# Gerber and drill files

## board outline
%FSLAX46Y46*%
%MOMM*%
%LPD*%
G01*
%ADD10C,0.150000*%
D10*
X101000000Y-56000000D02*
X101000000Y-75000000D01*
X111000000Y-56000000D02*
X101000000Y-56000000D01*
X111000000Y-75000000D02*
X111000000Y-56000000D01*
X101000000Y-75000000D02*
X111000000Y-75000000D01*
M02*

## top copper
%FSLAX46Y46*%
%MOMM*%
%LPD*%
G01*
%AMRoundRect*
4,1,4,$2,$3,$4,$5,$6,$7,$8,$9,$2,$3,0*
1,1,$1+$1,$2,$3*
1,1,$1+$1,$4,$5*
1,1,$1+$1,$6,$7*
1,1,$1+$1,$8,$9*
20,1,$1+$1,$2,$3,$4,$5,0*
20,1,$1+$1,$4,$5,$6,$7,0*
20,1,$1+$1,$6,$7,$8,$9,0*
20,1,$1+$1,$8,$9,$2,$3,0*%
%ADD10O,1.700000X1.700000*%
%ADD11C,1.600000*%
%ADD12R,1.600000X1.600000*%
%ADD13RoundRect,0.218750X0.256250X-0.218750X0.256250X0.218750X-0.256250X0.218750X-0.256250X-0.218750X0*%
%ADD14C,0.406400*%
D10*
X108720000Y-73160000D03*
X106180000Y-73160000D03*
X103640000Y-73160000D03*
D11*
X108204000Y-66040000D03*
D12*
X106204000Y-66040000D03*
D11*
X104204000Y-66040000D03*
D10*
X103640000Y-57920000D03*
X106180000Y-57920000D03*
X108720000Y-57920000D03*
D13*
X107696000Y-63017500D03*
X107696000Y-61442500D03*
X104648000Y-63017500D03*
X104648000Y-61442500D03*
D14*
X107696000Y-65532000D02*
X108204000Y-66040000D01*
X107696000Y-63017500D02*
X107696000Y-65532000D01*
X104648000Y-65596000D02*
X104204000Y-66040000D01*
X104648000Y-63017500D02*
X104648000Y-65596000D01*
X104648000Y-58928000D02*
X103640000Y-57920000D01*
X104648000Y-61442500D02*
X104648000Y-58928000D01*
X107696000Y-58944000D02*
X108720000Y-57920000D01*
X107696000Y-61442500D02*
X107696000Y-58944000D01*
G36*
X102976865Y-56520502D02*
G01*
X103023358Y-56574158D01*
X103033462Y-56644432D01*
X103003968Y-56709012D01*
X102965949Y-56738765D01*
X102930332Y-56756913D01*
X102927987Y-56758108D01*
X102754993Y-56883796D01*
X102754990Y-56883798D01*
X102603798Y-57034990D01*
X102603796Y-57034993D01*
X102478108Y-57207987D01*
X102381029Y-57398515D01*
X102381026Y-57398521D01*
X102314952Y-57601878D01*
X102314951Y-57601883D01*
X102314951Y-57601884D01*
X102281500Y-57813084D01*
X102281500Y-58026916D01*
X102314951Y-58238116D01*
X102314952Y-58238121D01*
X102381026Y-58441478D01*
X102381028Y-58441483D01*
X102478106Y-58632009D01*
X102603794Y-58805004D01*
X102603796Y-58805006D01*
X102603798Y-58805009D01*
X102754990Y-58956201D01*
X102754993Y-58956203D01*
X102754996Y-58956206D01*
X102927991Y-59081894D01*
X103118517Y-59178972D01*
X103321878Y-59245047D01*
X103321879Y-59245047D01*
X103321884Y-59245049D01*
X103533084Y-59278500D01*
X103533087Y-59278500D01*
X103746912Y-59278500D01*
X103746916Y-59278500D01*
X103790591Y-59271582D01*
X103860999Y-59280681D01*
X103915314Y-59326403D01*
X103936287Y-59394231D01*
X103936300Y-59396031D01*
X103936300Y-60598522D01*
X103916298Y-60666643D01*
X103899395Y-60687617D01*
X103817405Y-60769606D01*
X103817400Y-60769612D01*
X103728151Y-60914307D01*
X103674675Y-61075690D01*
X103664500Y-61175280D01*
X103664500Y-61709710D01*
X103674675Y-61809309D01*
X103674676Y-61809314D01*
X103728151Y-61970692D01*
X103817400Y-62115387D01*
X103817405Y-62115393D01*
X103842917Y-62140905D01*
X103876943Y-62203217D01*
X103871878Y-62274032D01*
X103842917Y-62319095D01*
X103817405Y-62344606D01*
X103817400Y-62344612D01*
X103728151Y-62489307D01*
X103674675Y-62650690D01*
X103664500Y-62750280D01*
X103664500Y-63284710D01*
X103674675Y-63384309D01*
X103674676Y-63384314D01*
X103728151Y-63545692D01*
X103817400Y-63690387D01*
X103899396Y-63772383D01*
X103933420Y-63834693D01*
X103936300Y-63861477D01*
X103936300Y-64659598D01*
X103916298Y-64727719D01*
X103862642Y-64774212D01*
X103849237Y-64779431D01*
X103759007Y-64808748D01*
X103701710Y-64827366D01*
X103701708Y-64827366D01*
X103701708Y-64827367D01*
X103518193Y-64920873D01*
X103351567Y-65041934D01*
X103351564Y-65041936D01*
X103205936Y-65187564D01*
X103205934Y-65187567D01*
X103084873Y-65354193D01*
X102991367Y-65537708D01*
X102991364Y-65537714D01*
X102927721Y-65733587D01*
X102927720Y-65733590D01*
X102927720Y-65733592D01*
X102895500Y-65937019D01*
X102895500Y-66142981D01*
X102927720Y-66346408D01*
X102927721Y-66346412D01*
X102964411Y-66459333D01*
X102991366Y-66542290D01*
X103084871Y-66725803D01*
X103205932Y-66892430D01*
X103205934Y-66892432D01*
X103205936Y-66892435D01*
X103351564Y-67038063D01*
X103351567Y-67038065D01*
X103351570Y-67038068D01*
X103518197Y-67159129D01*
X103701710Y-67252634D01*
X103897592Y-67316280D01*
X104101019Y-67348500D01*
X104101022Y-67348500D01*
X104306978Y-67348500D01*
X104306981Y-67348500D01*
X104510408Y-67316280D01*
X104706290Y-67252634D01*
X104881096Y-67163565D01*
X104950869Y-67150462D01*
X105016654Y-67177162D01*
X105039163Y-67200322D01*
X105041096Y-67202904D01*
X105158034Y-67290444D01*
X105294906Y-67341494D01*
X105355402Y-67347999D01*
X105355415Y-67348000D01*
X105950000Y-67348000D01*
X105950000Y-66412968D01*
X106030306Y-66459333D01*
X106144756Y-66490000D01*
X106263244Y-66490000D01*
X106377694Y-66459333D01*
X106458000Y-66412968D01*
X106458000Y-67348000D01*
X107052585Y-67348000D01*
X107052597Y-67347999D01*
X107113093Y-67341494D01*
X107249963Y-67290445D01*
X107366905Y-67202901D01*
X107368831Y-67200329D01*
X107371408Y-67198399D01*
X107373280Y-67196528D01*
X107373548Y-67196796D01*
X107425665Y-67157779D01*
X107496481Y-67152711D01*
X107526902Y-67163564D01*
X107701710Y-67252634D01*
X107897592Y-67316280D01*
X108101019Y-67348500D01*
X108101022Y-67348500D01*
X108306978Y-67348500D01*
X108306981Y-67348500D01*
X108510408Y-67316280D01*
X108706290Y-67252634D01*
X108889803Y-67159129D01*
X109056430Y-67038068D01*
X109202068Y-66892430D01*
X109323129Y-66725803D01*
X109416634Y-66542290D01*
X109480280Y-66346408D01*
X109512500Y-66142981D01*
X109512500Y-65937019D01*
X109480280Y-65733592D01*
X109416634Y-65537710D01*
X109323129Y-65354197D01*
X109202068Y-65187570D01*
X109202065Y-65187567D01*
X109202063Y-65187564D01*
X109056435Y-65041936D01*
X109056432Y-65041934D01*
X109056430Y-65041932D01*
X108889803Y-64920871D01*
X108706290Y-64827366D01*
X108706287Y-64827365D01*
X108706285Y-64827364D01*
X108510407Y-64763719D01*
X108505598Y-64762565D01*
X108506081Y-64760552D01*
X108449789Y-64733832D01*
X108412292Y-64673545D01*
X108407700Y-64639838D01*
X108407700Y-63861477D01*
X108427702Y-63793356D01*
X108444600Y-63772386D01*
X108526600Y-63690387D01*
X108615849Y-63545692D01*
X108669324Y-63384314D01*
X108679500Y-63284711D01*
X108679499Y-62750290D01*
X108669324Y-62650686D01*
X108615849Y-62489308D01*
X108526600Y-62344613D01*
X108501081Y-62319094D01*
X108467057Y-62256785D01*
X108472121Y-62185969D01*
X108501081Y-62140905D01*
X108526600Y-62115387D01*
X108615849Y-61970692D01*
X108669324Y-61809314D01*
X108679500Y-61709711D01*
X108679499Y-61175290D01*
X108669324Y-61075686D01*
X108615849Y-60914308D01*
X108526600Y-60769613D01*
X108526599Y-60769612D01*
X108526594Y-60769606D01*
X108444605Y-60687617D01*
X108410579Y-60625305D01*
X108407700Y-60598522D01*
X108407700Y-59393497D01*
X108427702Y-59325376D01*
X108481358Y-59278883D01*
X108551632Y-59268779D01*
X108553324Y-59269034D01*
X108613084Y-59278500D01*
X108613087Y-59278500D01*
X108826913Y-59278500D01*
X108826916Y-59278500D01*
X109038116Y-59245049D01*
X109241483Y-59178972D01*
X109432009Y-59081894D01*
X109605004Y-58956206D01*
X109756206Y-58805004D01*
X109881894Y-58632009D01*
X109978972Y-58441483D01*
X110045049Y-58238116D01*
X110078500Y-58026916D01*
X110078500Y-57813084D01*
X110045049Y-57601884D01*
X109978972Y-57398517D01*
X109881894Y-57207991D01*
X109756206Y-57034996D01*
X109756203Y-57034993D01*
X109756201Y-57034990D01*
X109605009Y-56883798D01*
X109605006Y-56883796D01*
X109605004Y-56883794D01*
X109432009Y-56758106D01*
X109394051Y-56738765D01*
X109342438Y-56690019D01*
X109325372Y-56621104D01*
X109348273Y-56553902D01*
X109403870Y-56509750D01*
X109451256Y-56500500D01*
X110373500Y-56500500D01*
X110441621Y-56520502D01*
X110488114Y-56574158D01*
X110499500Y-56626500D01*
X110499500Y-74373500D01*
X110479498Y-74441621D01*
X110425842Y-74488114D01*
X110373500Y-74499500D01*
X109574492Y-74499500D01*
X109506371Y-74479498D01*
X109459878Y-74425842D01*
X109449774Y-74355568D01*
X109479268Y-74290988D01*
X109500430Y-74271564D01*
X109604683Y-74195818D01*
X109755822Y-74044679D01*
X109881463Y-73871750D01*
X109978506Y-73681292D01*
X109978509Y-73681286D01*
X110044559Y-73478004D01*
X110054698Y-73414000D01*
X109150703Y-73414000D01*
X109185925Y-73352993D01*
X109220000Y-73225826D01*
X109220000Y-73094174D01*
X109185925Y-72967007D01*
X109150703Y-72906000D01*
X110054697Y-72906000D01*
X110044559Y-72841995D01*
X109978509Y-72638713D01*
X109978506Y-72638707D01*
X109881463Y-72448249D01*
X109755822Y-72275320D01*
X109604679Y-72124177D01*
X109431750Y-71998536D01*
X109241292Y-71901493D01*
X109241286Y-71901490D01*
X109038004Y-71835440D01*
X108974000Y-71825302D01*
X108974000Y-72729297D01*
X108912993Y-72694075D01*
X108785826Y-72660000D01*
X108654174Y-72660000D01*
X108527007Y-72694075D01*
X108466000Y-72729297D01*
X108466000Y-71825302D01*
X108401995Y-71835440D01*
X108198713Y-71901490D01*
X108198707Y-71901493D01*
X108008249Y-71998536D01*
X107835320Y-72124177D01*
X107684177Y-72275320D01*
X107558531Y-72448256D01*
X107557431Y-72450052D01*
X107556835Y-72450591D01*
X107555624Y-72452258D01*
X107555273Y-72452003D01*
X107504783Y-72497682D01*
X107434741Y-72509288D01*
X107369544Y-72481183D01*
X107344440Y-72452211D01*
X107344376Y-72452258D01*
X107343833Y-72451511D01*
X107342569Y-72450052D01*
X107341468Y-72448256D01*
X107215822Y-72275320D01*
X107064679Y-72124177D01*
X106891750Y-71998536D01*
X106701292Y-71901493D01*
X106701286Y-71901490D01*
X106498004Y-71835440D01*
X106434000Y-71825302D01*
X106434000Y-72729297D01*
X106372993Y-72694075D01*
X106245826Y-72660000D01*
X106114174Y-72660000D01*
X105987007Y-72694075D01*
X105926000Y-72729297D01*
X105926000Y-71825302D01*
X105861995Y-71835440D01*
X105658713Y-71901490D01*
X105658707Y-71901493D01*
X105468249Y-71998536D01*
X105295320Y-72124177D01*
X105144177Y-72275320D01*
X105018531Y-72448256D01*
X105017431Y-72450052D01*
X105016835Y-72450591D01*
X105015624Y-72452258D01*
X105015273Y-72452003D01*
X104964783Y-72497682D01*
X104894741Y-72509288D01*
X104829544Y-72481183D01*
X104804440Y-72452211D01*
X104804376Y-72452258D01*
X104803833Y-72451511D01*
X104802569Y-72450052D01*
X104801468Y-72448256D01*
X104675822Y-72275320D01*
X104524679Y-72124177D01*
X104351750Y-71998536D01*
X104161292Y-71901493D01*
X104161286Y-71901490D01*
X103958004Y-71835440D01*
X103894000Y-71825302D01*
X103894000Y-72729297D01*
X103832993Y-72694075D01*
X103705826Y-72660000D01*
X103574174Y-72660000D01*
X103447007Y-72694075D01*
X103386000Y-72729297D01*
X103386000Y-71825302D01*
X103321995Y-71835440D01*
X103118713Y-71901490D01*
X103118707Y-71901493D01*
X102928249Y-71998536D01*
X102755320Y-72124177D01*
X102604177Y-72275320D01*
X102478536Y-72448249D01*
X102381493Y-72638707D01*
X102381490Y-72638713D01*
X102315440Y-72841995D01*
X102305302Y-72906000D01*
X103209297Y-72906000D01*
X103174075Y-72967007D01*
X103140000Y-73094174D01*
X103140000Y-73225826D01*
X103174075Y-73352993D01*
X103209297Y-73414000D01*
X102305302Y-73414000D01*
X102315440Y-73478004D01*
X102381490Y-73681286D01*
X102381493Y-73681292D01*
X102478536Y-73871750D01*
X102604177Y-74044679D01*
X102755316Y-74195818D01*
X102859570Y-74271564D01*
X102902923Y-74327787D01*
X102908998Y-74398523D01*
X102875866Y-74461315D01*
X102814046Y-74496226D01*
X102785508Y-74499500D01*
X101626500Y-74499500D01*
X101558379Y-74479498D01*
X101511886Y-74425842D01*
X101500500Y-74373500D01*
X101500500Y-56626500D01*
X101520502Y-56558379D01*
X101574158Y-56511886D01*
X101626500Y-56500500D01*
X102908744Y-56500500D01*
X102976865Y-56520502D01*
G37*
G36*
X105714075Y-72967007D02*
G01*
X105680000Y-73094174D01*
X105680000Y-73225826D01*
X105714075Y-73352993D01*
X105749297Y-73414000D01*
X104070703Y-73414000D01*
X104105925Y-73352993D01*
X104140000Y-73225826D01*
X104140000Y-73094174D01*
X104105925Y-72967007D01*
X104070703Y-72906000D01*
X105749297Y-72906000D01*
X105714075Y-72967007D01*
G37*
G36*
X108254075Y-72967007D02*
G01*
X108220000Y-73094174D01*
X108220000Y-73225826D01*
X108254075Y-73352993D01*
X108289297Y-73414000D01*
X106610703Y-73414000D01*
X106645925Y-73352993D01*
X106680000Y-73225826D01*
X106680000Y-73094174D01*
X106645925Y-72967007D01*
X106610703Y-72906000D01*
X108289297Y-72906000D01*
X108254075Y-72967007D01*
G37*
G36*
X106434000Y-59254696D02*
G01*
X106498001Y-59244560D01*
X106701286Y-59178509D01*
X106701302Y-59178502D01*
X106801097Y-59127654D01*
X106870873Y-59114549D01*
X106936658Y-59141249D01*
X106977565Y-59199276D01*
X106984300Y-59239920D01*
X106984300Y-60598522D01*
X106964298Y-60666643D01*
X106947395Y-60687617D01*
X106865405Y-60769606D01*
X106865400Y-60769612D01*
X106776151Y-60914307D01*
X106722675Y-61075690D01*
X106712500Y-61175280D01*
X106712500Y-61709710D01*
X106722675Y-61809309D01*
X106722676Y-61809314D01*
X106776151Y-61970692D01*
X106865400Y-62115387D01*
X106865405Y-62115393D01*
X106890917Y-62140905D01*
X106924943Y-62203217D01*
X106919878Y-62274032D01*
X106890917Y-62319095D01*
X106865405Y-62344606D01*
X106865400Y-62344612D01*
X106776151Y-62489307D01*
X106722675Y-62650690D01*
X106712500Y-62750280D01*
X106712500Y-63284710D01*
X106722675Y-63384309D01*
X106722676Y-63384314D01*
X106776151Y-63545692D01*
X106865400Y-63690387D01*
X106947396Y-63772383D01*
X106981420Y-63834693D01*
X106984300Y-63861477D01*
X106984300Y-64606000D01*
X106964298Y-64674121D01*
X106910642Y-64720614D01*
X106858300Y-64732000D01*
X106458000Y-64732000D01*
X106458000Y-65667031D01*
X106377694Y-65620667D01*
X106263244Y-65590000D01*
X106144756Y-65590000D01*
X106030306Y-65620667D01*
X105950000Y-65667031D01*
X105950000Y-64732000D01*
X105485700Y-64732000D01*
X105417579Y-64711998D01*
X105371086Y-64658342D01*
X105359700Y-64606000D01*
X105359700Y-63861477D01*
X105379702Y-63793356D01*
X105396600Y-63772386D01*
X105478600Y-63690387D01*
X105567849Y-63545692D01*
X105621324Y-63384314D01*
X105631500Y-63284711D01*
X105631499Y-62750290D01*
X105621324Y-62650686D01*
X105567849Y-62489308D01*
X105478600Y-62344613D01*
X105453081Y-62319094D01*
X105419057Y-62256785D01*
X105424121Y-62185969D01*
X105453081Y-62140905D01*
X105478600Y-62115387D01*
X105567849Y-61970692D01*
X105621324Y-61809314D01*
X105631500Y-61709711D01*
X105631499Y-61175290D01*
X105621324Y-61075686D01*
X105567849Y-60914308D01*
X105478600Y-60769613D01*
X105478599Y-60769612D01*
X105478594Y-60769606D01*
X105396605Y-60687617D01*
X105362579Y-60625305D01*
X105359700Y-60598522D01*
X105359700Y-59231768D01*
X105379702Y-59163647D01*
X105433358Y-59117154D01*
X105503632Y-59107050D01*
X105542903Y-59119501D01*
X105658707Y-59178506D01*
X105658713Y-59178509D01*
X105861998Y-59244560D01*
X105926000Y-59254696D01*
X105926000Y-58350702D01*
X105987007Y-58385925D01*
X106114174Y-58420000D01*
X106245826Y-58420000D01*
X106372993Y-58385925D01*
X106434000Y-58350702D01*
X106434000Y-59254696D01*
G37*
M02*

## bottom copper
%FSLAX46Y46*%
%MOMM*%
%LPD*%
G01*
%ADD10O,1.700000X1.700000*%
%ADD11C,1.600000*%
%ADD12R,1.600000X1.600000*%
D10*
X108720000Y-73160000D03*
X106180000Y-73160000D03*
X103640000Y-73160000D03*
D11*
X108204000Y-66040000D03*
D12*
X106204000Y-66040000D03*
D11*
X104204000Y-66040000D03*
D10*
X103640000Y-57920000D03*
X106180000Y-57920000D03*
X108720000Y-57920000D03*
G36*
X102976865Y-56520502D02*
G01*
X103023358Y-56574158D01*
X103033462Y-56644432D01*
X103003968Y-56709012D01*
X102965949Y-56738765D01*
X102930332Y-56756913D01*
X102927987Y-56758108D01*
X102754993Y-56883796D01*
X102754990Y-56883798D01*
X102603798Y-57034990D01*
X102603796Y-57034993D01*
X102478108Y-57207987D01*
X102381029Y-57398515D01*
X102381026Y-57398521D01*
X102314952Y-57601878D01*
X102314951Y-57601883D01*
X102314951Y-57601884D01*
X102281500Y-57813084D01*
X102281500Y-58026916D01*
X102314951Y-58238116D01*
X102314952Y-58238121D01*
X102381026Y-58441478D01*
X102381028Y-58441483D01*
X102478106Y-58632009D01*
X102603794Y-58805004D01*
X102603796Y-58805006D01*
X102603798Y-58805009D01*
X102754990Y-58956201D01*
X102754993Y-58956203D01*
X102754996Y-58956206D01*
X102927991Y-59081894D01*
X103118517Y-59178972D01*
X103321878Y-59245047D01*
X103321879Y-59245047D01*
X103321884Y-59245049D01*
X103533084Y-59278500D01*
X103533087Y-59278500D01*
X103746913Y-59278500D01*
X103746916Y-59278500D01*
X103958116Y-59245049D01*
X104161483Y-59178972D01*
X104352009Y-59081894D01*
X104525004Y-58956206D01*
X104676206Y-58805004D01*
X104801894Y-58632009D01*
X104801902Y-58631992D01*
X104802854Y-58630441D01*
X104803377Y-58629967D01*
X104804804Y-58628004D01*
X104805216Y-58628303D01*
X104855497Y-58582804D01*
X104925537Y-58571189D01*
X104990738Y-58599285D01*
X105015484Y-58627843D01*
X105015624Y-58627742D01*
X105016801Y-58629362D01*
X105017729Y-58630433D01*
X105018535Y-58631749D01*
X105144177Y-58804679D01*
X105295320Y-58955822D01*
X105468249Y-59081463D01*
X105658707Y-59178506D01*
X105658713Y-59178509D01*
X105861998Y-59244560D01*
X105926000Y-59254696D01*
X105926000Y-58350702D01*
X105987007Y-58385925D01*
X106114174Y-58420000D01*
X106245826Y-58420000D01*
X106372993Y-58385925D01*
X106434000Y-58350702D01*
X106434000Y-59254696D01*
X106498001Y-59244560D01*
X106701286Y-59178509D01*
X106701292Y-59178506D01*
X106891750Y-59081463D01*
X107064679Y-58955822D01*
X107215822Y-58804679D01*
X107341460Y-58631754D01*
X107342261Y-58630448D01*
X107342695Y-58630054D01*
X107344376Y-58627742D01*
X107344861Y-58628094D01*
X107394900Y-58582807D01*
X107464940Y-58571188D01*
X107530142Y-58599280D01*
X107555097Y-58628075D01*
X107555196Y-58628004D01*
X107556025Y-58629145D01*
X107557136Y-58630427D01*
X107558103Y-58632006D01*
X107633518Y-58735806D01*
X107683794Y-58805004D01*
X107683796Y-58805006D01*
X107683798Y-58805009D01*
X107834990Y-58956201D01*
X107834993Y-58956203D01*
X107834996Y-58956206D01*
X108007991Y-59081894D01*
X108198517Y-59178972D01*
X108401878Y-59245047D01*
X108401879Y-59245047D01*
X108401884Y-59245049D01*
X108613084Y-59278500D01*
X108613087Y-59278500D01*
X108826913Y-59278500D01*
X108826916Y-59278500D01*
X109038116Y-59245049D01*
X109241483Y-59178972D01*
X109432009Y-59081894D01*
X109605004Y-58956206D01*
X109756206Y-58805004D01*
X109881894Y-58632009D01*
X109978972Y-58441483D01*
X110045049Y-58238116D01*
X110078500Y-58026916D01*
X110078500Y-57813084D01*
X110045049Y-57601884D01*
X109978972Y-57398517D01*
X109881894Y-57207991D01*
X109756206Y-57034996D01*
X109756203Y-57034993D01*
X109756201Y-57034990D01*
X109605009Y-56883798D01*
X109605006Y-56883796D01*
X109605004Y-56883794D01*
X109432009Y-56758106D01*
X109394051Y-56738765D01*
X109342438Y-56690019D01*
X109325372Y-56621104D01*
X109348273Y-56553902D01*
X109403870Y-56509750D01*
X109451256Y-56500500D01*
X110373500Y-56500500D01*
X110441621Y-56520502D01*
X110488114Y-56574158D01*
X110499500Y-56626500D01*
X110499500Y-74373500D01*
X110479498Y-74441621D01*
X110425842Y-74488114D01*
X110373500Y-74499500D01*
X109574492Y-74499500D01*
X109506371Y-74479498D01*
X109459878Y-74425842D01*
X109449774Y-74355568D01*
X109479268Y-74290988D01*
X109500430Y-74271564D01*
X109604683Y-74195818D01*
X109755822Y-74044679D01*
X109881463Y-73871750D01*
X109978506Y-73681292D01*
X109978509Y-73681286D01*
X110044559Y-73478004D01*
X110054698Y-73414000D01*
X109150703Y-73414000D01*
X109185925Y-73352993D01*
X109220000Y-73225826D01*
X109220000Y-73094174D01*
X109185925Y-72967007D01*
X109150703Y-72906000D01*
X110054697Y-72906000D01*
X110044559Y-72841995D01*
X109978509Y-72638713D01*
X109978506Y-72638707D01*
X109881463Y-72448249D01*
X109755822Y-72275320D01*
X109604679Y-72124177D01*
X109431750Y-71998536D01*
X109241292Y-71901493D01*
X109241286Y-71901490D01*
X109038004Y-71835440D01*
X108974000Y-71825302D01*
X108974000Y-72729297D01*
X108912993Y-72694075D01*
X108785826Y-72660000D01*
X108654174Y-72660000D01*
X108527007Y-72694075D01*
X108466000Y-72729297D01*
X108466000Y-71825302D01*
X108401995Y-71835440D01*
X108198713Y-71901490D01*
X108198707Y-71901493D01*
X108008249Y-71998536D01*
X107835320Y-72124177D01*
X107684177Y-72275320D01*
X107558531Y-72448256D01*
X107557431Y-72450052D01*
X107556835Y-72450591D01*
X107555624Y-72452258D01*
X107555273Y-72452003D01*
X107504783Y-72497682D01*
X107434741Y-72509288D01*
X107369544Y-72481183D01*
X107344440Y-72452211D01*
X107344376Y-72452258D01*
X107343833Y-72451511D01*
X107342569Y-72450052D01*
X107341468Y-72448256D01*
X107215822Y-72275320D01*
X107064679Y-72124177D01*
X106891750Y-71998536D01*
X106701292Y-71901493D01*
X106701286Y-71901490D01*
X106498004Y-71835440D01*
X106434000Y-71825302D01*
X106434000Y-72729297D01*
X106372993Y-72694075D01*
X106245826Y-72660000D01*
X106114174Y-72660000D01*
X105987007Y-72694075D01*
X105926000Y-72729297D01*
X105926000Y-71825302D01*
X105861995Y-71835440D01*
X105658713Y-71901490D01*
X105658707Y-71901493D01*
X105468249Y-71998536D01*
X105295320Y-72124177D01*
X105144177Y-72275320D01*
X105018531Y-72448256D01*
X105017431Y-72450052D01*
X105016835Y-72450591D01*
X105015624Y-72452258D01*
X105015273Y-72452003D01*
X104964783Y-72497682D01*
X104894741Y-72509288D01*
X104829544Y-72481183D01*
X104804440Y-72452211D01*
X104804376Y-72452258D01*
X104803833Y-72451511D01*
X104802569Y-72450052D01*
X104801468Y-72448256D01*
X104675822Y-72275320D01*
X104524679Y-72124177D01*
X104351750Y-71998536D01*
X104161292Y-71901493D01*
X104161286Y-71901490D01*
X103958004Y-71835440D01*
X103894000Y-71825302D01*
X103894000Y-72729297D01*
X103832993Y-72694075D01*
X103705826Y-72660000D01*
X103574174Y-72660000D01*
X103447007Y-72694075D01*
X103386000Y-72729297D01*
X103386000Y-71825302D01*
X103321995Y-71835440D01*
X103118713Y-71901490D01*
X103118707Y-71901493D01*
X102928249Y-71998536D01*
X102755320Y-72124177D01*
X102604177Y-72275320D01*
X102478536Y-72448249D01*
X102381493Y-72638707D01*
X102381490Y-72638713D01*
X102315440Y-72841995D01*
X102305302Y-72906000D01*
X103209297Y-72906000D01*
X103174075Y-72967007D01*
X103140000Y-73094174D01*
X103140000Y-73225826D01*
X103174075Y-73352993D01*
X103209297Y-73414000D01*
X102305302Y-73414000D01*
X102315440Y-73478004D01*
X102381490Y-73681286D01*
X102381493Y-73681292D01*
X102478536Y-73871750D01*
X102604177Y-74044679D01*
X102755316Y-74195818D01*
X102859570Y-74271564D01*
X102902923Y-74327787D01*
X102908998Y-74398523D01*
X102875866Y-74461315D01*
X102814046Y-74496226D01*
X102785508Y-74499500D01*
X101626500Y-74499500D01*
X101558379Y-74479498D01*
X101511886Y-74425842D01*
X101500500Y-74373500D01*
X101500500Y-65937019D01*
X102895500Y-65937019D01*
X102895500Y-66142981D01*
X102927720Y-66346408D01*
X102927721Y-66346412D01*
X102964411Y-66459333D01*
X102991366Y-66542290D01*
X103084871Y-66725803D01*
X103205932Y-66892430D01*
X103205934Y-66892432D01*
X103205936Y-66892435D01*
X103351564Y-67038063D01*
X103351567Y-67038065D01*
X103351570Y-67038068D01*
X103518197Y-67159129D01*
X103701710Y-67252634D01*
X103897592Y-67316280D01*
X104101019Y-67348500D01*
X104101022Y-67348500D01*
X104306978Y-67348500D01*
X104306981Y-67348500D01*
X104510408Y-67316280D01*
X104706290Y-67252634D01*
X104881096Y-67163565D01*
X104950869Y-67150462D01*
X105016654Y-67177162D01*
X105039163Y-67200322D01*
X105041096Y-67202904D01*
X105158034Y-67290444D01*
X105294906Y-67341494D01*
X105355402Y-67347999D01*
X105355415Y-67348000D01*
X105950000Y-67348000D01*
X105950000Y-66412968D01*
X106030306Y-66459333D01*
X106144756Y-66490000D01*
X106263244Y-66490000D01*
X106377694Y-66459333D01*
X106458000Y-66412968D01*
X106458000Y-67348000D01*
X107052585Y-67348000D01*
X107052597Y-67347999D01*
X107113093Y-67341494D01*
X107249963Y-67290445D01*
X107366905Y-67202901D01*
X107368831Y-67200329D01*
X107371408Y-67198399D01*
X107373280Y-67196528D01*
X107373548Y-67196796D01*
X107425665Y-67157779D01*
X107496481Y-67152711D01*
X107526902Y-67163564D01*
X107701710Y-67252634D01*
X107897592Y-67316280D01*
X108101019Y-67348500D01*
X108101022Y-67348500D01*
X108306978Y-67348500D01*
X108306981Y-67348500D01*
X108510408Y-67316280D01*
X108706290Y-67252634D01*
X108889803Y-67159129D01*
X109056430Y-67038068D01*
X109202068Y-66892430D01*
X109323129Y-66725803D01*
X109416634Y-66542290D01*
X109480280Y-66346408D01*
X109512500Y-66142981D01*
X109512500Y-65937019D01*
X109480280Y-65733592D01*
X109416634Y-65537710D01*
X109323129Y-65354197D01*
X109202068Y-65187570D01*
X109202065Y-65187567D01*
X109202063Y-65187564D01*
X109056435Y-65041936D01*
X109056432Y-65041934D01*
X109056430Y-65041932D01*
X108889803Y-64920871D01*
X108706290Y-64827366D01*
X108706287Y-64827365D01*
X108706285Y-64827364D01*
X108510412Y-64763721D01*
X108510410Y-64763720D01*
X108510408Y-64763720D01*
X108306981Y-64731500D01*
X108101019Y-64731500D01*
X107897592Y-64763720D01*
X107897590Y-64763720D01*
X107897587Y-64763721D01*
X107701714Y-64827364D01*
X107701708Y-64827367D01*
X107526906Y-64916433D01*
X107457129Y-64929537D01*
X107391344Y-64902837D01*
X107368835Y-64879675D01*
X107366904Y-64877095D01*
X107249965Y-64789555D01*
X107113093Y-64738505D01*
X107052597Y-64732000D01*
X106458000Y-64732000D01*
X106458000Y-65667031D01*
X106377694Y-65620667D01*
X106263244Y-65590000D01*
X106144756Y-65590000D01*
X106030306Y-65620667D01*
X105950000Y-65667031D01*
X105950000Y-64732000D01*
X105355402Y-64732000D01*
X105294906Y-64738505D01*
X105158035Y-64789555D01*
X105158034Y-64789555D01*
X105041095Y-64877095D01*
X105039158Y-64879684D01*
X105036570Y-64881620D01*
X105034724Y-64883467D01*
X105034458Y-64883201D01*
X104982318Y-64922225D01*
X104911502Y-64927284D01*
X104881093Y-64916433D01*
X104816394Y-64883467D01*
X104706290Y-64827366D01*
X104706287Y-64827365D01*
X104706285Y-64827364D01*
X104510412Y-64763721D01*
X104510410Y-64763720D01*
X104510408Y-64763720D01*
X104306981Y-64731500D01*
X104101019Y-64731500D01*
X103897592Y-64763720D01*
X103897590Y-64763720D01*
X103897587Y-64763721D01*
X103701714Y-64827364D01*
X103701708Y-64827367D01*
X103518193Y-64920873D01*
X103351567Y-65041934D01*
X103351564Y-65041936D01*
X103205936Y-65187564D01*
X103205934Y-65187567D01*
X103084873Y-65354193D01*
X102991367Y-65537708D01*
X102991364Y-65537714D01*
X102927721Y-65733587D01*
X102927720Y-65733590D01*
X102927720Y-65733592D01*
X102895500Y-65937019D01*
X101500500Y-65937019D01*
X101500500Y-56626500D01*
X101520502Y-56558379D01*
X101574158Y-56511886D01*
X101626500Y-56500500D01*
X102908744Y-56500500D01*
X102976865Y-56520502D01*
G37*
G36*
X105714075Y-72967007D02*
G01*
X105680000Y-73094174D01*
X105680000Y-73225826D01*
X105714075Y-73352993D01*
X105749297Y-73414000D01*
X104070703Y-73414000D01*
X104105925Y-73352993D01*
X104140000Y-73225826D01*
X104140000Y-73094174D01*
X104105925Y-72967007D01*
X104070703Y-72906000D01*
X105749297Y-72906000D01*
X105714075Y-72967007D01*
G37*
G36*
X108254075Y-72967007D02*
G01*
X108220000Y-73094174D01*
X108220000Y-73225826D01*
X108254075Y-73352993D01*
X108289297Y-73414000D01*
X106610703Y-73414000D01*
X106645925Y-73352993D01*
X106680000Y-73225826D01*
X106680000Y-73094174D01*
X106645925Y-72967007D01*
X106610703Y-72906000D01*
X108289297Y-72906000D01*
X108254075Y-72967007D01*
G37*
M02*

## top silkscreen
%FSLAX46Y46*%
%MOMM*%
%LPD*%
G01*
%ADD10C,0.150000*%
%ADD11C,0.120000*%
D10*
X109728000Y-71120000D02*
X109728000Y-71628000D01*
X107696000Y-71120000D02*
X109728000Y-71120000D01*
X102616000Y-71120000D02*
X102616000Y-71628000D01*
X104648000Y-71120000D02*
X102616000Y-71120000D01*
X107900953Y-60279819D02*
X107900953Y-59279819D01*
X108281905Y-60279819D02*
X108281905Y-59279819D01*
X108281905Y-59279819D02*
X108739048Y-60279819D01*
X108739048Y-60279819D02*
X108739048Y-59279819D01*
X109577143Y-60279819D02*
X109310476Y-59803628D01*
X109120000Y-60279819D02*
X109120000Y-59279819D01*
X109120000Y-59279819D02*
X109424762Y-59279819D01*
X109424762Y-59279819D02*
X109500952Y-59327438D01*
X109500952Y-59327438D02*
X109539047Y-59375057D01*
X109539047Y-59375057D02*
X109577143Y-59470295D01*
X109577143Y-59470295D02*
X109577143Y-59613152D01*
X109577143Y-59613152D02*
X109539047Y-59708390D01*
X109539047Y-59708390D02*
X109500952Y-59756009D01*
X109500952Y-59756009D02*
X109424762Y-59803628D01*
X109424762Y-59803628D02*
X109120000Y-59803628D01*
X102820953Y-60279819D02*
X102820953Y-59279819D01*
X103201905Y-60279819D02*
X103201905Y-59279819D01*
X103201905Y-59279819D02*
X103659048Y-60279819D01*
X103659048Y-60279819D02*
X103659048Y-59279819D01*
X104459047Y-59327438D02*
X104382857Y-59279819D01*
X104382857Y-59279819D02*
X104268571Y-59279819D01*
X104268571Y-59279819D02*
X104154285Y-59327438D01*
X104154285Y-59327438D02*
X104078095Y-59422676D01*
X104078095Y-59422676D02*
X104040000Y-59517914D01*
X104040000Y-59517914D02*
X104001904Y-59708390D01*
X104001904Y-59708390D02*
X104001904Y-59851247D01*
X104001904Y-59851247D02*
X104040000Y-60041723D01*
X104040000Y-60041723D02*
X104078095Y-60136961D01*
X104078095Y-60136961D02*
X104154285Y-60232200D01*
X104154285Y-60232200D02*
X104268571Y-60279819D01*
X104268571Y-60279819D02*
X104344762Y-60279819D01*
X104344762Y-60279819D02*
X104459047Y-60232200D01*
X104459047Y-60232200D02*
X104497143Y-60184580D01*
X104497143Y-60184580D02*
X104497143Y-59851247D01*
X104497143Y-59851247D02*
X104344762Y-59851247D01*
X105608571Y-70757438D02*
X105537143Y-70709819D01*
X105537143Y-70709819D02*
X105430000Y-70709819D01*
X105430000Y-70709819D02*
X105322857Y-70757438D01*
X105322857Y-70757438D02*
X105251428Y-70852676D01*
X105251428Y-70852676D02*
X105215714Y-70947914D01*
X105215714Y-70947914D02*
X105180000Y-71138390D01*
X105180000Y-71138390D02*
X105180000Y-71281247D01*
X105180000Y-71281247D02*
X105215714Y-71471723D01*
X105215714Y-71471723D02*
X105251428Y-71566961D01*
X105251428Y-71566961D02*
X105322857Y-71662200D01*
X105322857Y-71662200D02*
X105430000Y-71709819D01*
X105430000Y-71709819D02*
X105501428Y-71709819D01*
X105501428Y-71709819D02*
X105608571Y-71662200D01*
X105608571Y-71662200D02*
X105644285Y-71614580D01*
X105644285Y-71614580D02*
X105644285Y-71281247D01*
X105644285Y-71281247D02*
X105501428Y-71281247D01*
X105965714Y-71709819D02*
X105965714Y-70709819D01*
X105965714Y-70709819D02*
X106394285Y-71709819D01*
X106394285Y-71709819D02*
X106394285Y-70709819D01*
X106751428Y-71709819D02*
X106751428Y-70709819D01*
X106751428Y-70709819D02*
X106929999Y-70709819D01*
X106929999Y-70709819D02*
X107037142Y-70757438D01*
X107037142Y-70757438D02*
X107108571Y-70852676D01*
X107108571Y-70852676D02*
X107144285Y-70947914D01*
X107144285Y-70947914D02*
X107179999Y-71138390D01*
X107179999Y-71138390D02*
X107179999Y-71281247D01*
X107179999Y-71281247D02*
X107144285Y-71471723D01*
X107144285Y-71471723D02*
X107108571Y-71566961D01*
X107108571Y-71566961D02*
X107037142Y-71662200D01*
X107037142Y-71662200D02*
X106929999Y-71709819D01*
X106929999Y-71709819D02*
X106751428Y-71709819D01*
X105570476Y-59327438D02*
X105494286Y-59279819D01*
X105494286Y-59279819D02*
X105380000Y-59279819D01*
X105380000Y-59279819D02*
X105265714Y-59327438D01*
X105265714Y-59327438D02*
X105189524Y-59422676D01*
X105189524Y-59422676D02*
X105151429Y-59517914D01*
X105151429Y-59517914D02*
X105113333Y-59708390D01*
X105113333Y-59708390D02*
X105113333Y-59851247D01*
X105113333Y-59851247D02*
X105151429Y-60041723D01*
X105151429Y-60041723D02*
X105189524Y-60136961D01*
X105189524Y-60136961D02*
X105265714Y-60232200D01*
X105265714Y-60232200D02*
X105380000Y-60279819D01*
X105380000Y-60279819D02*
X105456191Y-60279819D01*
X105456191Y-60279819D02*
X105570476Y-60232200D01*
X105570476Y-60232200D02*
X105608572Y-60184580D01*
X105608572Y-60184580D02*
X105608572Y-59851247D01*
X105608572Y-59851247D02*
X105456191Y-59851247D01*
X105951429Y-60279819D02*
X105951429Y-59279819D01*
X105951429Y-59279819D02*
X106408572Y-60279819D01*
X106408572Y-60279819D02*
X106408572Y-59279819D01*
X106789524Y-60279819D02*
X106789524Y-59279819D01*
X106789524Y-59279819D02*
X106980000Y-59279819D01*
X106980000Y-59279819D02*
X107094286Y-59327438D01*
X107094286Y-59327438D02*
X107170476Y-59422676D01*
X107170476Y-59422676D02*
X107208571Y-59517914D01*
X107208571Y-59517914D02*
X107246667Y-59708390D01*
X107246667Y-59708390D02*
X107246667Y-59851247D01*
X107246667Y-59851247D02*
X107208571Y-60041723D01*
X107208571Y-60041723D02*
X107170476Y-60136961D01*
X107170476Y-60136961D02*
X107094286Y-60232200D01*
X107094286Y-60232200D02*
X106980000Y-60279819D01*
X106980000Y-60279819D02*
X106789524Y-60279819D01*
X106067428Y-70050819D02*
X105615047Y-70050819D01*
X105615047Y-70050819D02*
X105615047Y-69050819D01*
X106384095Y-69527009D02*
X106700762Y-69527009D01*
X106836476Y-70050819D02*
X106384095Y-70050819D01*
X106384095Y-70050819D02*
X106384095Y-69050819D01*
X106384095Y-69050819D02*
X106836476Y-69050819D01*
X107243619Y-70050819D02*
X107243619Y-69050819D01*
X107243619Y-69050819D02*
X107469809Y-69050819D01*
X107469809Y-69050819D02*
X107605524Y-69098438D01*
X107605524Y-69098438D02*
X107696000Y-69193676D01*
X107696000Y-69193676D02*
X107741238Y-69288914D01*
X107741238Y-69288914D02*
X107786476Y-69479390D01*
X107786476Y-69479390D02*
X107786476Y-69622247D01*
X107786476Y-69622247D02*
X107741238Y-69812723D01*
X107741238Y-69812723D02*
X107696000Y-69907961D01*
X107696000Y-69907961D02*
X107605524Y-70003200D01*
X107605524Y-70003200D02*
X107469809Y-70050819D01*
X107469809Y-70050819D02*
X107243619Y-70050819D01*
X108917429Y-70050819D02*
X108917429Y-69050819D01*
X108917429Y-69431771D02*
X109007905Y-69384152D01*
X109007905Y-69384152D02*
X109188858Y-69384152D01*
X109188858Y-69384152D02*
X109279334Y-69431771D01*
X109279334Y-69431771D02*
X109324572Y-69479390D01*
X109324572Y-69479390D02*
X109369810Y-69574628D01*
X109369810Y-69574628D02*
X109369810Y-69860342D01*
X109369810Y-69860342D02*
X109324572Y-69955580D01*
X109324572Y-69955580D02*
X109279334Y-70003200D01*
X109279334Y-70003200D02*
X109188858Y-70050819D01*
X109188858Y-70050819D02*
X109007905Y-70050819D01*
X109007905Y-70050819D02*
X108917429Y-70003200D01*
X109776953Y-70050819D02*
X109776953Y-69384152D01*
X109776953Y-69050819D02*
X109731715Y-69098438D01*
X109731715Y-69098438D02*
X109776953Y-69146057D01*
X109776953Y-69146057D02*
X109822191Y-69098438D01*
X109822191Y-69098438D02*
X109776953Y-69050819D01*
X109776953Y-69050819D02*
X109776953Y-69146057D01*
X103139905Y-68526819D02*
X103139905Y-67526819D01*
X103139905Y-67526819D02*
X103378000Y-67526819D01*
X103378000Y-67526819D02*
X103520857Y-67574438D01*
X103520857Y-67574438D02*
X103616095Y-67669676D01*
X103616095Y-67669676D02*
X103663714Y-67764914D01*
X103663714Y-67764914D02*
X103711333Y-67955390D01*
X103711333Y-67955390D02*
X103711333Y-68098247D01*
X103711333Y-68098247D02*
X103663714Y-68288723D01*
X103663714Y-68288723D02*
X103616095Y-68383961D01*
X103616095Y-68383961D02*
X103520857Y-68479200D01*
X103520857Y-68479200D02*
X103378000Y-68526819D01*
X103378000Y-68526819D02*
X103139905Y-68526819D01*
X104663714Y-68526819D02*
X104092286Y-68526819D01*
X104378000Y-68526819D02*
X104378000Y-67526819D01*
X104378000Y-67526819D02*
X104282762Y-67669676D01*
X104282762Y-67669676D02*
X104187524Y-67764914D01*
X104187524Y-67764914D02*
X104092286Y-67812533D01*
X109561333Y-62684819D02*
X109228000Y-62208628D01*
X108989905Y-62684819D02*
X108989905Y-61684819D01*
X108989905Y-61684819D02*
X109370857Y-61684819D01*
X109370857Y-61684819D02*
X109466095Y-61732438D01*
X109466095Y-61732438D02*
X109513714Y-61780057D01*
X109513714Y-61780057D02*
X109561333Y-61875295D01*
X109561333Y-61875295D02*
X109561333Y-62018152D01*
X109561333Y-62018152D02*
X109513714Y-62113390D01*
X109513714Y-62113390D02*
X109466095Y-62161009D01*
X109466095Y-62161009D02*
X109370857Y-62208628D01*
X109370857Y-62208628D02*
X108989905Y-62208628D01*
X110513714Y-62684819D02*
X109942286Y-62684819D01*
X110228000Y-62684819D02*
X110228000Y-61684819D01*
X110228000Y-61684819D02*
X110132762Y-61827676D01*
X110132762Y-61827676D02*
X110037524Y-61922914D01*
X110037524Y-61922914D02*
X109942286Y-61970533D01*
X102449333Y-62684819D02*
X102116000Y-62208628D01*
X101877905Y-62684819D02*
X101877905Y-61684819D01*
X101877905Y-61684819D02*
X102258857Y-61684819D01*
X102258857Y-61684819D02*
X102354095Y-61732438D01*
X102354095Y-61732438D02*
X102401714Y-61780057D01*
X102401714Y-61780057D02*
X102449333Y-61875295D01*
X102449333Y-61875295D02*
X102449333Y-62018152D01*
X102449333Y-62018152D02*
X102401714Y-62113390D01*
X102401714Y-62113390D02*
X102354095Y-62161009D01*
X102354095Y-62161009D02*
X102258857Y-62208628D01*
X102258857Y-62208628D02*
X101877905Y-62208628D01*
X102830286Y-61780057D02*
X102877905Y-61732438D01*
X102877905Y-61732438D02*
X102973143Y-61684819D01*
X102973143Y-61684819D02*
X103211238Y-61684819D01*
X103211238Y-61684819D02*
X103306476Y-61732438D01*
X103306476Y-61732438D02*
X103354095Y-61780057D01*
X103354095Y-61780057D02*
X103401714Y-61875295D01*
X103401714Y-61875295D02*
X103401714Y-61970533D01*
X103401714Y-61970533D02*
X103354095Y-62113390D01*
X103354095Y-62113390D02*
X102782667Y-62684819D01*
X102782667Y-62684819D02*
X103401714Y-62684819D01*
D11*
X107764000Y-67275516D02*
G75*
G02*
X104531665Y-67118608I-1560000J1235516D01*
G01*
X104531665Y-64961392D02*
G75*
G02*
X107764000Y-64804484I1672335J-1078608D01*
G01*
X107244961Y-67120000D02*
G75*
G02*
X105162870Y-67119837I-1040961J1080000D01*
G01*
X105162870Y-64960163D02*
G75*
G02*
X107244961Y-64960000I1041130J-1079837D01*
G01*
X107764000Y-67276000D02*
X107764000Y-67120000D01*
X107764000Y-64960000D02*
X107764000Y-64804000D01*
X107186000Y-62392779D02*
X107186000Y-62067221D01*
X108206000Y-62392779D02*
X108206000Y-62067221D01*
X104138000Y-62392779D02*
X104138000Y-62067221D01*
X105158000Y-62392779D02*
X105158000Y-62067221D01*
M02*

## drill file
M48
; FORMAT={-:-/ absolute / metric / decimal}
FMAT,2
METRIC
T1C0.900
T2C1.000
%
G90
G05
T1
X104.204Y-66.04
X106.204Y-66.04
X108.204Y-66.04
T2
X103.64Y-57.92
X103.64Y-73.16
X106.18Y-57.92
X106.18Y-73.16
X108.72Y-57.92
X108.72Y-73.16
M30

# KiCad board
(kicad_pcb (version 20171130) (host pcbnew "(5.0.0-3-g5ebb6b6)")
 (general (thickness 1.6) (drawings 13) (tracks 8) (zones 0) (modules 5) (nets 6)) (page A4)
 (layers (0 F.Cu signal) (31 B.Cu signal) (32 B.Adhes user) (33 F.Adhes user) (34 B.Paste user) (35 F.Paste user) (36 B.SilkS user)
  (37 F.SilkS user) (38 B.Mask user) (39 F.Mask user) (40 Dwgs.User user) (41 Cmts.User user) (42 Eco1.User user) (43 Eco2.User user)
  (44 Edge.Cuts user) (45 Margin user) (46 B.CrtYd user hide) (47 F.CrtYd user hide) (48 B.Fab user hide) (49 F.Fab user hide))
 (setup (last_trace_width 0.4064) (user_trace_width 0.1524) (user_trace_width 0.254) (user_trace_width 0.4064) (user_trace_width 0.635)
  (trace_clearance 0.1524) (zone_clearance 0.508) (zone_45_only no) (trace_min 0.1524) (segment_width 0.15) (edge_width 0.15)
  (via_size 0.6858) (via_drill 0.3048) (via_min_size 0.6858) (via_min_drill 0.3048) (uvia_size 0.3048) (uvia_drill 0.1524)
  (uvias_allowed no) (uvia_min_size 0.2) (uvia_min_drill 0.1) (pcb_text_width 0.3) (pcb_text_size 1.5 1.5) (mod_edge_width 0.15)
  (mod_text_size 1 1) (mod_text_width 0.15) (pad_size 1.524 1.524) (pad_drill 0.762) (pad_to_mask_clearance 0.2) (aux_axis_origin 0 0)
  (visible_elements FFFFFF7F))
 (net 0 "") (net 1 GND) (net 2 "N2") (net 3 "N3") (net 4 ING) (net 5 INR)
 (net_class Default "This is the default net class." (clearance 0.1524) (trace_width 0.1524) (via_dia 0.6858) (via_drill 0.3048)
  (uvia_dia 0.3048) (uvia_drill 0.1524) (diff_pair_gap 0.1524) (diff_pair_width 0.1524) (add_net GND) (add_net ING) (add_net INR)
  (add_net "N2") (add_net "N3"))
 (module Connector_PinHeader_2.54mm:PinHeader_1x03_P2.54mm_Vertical (layer B.Cu) (at 103.64 73.16 270)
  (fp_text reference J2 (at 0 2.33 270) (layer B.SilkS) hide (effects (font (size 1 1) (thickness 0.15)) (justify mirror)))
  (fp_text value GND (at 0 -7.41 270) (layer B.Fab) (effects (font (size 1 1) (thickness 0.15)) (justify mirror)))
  (pad 3 thru_hole oval (at 0 -5.08 270) (size 1.7 1.7) (drill 1) (layers *.Cu *.Mask) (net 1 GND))
  (pad 2 thru_hole oval (at 0 -2.54 270) (size 1.7 1.7) (drill 1) (layers *.Cu *.Mask) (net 1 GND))
  (pad 1 thru_hole oval (at 0 0 270) (size 1.7 1.7) (drill 1) (layers *.Cu *.Mask) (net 1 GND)))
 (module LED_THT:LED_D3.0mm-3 (layer F.Cu) (at 108.704 66.04 180)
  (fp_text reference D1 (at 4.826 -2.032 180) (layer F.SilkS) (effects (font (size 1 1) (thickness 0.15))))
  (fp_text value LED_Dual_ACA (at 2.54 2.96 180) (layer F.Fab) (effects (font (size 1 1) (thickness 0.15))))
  (fp_arc (start 2.5 0) (end 0.94 -1.235516) (angle 108.8) (layer F.SilkS) (width 0.12))
  (fp_arc (start 2.5 0) (end 0.94 1.235516) (angle -108.8) (layer F.SilkS) (width 0.12))
  (fp_arc (start 2.5 0) (end 1.459039 -1.08) (angle 87.9) (layer F.SilkS) (width 0.12))
  (fp_arc (start 2.5 0) (end 1.459039 1.08) (angle -87.9) (layer F.SilkS) (width 0.12))
  (fp_line (start 0.94 -1.236) (end 0.94 -1.08) (layer F.SilkS) (width 0.12))
  (fp_line (start 0.94 1.08) (end 0.94 1.236) (layer F.SilkS) (width 0.12))
  (pad 1 thru_hole circle (at 0.5 0 180) (size 1.6 1.6) (drill 0.9) (layers *.Cu *.Mask) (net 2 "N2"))
  (pad 2 thru_hole rect (at 2.5 0 180) (size 1.6 1.6) (drill 0.9) (layers *.Cu *.Mask) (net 1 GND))
  (pad 3 thru_hole circle (at 4.5 0 180) (size 1.6 1.6) (drill 0.9) (layers *.Cu *.Mask) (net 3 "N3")))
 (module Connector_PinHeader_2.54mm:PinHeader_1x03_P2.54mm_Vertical (layer B.Cu) (at 103.64 57.92 270)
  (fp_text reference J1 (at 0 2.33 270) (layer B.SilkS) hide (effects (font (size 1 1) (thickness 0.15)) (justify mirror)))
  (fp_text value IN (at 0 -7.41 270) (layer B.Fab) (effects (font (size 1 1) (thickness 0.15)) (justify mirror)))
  (pad 1 thru_hole oval (at 0 0 270) (size 1.7 1.7) (drill 1) (layers *.Cu *.Mask) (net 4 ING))
  (pad 2 thru_hole oval (at 0 -2.54 270) (size 1.7 1.7) (drill 1) (layers *.Cu *.Mask) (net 1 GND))
  (pad 3 thru_hole oval (at 0 -5.08 270) (size 1.7 1.7) (drill 1) (layers *.Cu *.Mask) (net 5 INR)))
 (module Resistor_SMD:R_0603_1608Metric (layer F.Cu) (at 107.696 62.23 90)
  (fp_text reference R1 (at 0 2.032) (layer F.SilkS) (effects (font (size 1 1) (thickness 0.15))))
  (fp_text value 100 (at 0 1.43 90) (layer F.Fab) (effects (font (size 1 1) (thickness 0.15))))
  (fp_line (start -0.162779 -0.51) (end 0.162779 -0.51) (layer F.SilkS) (width 0.12))
  (fp_line (start -0.162779 0.51) (end 0.162779 0.51) (layer F.SilkS) (width 0.12))
  (pad 1 smd roundrect (at -0.7875 0 90) (size 0.875 0.95) (layers F.Cu F.Paste F.Mask) (roundrect_rratio 0.25) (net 2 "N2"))
  (pad 2 smd roundrect (at 0.7875 0 90) (size 0.875 0.95) (layers F.Cu F.Paste F.Mask) (roundrect_rratio 0.25) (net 5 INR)))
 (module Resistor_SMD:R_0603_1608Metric (layer F.Cu) (at 104.648 62.23 90)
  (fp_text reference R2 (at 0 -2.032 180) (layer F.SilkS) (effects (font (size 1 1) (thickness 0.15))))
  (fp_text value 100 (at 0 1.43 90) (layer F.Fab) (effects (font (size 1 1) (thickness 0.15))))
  (fp_line (start -0.162779 -0.51) (end 0.162779 -0.51) (layer F.SilkS) (width 0.12))
  (fp_line (start -0.162779 0.51) (end 0.162779 0.51) (layer F.SilkS) (width 0.12))
  (pad 1 smd roundrect (at -0.7875 0 90) (size 0.875 0.95) (layers F.Cu F.Paste F.Mask) (roundrect_rratio 0.25) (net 3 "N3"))
  (pad 2 smd roundrect (at 0.7875 0 90) (size 0.875 0.95) (layers F.Cu F.Paste F.Mask) (roundrect_rratio 0.25) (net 4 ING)))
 (gr_line (start 109.728 71.12) (end 109.728 71.628) (layer F.SilkS) (width 0.15))
 (gr_line (start 107.696 71.12) (end 109.728 71.12) (layer F.SilkS) (width 0.15))
 (gr_line (start 102.616 71.12) (end 102.616 71.628) (layer F.SilkS) (width 0.15))
 (gr_line (start 104.648 71.12) (end 102.616 71.12) (layer F.SilkS) (width 0.15))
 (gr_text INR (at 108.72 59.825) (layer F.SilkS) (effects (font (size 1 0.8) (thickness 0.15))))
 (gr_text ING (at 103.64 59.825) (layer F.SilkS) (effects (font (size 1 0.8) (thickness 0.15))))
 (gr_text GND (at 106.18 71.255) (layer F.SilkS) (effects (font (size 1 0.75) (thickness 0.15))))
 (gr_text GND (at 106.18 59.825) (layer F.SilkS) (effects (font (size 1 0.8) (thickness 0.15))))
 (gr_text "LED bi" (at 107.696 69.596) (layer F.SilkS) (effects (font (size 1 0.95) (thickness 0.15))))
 (gr_line (start 101 56) (end 101 75) (layer Edge.Cuts) (width 0.15))
 (gr_line (start 111 56) (end 101 56) (layer Edge.Cuts) (width 0.15))
 (gr_line (start 111 75) (end 111 56) (layer Edge.Cuts) (width 0.15))
 (gr_line (start 101 75) (end 111 75) (layer Edge.Cuts) (width 0.15))
 (segment (start 107.696 65.532) (end 108.204 66.04) (width 0.4064) (layer F.Cu) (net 2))
 (segment (start 107.696 63.0175) (end 107.696 65.532) (width 0.4064) (layer F.Cu) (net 2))
 (segment (start 104.648 65.596) (end 104.204 66.04) (width 0.4064) (layer F.Cu) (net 3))
 (segment (start 104.648 63.0175) (end 104.648 65.596) (width 0.4064) (layer F.Cu) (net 3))
 (segment (start 104.648 58.928) (end 103.64 57.92) (width 0.4064) (layer F.Cu) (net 4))
 (segment (start 104.648 61.4425) (end 104.648 58.928) (width 0.4064) (layer F.Cu) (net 4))
 (segment (start 107.696 58.944) (end 108.72 57.92) (width 0.4064) (layer F.Cu) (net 5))
 (segment (start 107.696 61.4425) (end 107.696 58.944) (width 0.4064) (layer F.Cu) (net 5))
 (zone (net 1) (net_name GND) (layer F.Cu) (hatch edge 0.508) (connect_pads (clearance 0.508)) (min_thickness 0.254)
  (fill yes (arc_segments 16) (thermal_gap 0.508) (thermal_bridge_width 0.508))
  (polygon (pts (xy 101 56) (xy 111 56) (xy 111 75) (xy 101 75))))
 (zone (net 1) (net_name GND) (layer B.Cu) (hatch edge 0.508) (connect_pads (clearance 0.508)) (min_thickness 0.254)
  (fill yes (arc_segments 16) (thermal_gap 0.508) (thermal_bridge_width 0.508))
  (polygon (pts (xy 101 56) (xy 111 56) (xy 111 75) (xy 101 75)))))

